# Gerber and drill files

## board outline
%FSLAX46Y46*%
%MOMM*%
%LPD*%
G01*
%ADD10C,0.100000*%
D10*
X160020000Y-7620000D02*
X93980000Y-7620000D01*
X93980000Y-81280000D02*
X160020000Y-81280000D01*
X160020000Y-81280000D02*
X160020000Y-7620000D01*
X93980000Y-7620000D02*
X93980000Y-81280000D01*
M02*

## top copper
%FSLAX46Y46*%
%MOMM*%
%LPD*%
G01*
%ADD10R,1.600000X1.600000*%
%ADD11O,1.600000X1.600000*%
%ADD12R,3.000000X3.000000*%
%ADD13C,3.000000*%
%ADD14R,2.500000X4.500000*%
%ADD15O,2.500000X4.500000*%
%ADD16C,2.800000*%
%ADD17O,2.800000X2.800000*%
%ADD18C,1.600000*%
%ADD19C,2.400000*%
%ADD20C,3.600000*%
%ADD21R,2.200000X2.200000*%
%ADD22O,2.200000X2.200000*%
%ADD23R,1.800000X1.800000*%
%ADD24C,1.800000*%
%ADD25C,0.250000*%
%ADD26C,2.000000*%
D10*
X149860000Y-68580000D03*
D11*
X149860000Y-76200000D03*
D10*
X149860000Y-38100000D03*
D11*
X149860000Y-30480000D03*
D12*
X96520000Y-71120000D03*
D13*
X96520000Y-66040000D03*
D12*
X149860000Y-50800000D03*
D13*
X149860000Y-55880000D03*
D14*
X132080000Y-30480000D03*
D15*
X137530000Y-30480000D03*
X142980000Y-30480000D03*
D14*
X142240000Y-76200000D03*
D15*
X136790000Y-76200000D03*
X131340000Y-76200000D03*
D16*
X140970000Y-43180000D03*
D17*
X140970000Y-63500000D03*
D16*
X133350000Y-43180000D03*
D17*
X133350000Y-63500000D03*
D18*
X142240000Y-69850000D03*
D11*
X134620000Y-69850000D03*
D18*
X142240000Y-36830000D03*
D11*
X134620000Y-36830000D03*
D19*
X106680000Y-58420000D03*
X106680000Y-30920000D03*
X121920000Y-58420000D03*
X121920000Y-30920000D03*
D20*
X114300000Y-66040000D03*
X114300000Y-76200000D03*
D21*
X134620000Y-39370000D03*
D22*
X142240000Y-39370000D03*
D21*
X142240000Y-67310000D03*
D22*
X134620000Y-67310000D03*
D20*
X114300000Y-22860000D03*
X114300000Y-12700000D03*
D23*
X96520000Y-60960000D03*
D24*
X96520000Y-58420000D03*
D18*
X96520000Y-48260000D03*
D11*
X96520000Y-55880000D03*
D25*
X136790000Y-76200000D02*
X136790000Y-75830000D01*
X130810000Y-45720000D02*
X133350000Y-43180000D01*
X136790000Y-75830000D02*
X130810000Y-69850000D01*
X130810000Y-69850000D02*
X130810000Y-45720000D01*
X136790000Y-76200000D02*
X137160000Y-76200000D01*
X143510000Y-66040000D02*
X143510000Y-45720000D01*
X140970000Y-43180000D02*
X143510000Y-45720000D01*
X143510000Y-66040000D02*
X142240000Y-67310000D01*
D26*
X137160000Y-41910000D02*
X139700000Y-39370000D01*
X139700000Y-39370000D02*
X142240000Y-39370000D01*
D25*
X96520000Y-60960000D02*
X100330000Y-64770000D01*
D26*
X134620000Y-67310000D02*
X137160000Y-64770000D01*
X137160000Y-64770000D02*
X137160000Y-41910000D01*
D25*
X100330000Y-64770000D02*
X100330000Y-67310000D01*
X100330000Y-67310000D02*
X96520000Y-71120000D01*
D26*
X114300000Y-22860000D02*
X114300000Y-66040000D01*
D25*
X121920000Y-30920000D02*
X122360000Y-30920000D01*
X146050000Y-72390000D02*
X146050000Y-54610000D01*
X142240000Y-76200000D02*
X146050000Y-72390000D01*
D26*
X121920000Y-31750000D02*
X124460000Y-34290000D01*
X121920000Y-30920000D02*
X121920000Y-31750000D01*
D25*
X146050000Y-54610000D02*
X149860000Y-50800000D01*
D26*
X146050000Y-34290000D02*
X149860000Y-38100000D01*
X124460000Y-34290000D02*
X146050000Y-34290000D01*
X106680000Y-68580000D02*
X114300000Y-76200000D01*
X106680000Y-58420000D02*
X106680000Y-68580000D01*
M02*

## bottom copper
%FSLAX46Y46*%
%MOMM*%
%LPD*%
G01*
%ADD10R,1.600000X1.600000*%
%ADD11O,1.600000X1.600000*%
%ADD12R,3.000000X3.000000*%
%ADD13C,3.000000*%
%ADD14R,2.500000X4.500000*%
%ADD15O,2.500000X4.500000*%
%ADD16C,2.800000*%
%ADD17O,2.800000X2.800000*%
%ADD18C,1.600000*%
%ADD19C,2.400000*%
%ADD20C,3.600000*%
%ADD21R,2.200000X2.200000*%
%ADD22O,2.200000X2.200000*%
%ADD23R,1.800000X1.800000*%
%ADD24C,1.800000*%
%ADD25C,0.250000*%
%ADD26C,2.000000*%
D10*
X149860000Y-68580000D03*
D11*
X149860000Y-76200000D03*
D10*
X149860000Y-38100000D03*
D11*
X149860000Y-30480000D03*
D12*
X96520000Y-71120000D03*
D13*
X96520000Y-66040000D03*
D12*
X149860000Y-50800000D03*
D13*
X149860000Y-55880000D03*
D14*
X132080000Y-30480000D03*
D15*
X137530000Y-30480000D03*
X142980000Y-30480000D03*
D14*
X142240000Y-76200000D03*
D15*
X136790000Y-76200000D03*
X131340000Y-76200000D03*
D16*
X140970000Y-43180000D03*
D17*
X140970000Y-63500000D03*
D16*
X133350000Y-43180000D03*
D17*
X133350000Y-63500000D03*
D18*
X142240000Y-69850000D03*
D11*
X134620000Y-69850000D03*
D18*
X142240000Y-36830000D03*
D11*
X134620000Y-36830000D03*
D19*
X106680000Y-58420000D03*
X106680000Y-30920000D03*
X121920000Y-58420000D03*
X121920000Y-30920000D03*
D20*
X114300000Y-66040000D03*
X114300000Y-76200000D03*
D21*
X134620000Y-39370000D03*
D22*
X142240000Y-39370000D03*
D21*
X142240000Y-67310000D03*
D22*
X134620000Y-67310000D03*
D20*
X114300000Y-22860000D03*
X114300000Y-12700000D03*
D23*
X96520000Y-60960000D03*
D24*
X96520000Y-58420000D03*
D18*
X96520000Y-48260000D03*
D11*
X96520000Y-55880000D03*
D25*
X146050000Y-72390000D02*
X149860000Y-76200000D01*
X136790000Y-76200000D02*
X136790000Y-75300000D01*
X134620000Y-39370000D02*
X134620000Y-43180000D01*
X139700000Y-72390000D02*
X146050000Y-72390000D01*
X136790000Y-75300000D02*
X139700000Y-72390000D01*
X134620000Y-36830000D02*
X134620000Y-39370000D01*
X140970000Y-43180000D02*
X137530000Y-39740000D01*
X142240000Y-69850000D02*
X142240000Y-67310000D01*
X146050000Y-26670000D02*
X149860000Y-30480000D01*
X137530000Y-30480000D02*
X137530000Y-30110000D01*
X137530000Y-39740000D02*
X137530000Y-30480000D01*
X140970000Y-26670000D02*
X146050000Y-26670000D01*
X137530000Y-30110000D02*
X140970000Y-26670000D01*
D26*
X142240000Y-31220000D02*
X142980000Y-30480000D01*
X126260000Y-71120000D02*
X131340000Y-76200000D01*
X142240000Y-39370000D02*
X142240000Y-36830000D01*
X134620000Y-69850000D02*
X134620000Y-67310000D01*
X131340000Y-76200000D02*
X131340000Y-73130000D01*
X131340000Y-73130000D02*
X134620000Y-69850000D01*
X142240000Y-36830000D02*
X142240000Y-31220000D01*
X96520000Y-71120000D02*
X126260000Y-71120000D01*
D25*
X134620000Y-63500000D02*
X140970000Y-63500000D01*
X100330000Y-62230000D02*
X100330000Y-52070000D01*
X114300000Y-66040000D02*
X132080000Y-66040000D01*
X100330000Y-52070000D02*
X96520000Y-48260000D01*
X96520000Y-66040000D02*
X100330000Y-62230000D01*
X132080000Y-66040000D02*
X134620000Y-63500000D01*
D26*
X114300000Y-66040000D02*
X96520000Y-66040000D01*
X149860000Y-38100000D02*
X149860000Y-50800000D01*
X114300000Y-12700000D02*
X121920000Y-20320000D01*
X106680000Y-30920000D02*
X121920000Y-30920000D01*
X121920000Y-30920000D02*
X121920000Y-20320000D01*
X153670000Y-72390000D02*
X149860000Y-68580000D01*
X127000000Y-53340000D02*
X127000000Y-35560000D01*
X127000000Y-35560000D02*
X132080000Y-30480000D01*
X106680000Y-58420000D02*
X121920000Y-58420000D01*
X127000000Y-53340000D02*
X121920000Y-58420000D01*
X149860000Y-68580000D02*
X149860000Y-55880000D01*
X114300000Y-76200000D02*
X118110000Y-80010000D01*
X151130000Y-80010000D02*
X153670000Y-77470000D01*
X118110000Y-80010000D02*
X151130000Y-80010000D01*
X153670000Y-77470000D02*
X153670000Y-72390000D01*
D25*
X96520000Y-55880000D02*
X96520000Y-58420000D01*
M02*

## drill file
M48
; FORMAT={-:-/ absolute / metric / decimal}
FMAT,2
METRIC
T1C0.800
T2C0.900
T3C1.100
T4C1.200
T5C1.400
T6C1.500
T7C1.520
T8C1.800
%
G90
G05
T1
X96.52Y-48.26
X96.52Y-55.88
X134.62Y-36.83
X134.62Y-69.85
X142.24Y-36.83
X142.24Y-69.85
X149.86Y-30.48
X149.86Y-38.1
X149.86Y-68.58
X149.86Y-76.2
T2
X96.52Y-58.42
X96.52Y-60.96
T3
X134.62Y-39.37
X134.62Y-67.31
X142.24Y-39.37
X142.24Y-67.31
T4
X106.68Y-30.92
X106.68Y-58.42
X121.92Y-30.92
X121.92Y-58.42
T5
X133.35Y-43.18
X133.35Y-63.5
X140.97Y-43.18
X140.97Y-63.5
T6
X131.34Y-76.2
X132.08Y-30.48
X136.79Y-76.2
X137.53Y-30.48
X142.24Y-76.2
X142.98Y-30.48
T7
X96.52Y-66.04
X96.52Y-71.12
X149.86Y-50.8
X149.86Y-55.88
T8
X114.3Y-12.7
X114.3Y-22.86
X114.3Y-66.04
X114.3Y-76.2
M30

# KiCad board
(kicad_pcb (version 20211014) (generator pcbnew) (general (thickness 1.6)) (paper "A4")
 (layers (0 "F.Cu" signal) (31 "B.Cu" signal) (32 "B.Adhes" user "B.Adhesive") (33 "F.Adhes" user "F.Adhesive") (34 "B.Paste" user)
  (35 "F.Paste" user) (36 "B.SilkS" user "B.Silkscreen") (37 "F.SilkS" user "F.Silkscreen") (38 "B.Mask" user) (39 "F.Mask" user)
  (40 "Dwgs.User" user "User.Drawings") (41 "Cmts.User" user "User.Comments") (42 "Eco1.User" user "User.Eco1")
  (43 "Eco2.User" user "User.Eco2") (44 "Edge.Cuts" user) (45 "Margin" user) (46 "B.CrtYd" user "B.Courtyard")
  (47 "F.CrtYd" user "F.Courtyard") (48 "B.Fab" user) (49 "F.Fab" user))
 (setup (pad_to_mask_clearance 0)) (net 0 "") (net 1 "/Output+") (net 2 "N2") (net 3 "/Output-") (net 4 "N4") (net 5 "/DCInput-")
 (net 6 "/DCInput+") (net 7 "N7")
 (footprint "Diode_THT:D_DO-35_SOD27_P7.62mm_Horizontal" (layer "F.Cu") (at 149.86 68.58 -90)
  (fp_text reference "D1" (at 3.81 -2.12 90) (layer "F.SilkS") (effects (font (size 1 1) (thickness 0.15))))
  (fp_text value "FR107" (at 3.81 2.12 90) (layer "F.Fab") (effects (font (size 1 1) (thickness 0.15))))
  (pad "1" thru_hole rect (at 0 0 270) (size 1.6 1.6) (drill 0.8) (layers *.Cu *.Mask) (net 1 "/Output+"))
  (pad "2" thru_hole oval (at 7.62 0 270) (size 1.6 1.6) (drill 0.8) (layers *.Cu *.Mask) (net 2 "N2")))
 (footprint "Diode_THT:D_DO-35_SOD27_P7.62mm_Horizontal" (layer "F.Cu") (at 149.86 38.1 90)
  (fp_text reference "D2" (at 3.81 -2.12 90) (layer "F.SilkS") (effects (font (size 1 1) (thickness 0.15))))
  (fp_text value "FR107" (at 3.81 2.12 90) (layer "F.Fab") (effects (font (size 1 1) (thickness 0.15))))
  (pad "1" thru_hole rect (at 0 0 90) (size 1.6 1.6) (drill 0.8) (layers *.Cu *.Mask) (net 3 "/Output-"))
  (pad "2" thru_hole oval (at 7.62 0 90) (size 1.6 1.6) (drill 0.8) (layers *.Cu *.Mask) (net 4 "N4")))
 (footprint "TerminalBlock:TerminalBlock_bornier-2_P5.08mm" (layer "F.Cu") (at 96.52 71.12 90)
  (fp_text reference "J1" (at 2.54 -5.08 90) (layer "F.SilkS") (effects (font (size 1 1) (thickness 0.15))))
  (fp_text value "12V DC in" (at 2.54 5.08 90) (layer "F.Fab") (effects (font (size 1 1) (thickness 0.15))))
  (pad "1" thru_hole rect (at 0 0 90) (size 3 3) (drill 1.52) (layers *.Cu *.Mask) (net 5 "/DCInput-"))
  (pad "2" thru_hole circle (at 5.08 0 90) (size 3 3) (drill 1.52) (layers *.Cu *.Mask) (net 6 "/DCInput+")))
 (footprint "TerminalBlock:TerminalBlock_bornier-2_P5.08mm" (layer "F.Cu") (at 149.86 50.8 -90)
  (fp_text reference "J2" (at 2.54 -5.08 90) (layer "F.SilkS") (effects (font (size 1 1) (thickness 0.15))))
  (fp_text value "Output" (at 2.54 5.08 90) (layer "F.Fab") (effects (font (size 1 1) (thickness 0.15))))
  (pad "1" thru_hole rect (at 0 0 270) (size 3 3) (drill 1.52) (layers *.Cu *.Mask) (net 3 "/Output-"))
  (pad "2" thru_hole circle (at 5.08 0 270) (size 3 3) (drill 1.52) (layers *.Cu *.Mask) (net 1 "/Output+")))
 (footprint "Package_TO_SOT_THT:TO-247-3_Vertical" (layer "F.Cu") (at 132.08 30.48)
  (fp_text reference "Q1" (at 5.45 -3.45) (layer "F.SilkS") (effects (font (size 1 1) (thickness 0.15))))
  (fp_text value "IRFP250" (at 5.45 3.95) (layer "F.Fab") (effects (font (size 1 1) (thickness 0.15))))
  (pad "1" thru_hole rect (at 0 0) (size 2.5 4.5) (drill 1.5) (layers *.Cu *.Mask) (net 1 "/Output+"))
  (pad "2" thru_hole oval (at 5.45 0) (size 2.5 4.5) (drill 1.5) (layers *.Cu *.Mask) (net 4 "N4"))
  (pad "3" thru_hole oval (at 10.9 0) (size 2.5 4.5) (drill 1.5) (layers *.Cu *.Mask) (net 5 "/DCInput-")))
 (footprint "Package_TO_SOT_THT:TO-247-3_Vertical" (layer "F.Cu") (at 142.24 76.2 180)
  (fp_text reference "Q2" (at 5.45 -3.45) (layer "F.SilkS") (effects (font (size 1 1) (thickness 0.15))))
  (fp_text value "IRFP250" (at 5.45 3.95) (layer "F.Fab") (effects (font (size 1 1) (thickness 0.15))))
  (pad "1" thru_hole rect (at 0 0 180) (size 2.5 4.5) (drill 1.5) (layers *.Cu *.Mask) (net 3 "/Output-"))
  (pad "2" thru_hole oval (at 5.45 0 180) (size 2.5 4.5) (drill 1.5) (layers *.Cu *.Mask) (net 2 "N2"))
  (pad "3" thru_hole oval (at 10.9 0 180) (size 2.5 4.5) (drill 1.5) (layers *.Cu *.Mask) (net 5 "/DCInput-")))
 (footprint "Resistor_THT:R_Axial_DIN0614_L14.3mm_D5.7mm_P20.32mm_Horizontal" (layer "F.Cu") (at 140.97 43.18 -90)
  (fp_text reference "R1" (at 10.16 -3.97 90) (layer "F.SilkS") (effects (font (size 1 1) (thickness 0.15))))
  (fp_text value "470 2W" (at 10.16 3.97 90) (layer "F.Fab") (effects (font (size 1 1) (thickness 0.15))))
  (pad "1" thru_hole circle (at 0 0 270) (size 2.8 2.8) (drill 1.4) (layers *.Cu *.Mask) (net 4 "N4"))
  (pad "2" thru_hole oval (at 20.32 0 270) (size 2.8 2.8) (drill 1.4) (layers *.Cu *.Mask) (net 6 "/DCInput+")))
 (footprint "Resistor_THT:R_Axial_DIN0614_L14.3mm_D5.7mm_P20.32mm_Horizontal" (layer "F.Cu") (at 133.35 43.18 -90)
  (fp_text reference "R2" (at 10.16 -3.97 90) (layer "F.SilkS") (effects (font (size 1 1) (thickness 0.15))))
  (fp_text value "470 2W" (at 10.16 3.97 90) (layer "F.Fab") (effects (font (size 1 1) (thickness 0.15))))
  (pad "1" thru_hole circle (at 0 0 270) (size 2.8 2.8) (drill 1.4) (layers *.Cu *.Mask) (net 2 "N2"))
  (pad "2" thru_hole oval (at 20.32 0 270) (size 2.8 2.8) (drill 1.4) (layers *.Cu *.Mask) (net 6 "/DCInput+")))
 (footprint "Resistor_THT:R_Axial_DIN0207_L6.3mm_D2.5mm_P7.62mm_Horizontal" (layer "F.Cu") (at 142.24 69.85 180)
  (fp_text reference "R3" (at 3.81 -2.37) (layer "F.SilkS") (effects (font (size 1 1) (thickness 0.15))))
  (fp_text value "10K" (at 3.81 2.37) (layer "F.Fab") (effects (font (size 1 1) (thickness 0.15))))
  (pad "1" thru_hole circle (at 0 0 180) (size 1.6 1.6) (drill 0.8) (layers *.Cu *.Mask) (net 4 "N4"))
  (pad "2" thru_hole oval (at 7.62 0 180) (size 1.6 1.6) (drill 0.8) (layers *.Cu *.Mask) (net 5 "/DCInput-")))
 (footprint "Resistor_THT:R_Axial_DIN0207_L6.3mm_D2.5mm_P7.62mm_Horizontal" (layer "F.Cu") (at 142.24 36.83 180)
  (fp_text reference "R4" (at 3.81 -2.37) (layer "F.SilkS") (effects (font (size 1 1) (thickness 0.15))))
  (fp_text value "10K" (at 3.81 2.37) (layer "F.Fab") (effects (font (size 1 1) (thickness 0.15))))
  (pad "1" thru_hole circle (at 0 0 180) (size 1.6 1.6) (drill 0.8) (layers *.Cu *.Mask) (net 5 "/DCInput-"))
  (pad "2" thru_hole oval (at 7.62 0 180) (size 1.6 1.6) (drill 0.8) (layers *.Cu *.Mask) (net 2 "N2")))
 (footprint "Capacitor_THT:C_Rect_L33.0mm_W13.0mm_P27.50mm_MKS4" (layer "F.Cu") (at 106.68 58.42 90)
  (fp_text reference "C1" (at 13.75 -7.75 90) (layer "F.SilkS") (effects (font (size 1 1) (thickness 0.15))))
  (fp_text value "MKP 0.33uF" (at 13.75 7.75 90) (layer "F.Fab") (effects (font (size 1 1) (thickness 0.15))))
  (pad "1" thru_hole circle (at 0 0 90) (size 2.4 2.4) (drill 1.2) (layers *.Cu *.Mask) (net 1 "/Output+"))
  (pad "2" thru_hole circle (at 27.5 0 90) (size 2.4 2.4) (drill 1.2) (layers *.Cu *.Mask) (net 3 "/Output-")))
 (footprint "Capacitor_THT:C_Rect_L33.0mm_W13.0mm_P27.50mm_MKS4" (layer "F.Cu") (at 121.92 58.42 90)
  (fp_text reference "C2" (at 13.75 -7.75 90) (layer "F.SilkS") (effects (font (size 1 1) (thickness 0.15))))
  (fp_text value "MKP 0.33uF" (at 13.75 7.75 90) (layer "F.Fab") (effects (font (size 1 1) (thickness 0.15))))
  (pad "1" thru_hole circle (at 0 0 90) (size 2.4 2.4) (drill 1.2) (layers *.Cu *.Mask) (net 1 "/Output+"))
  (pad "2" thru_hole circle (at 27.5 0 90) (size 2.4 2.4) (drill 1.2) (layers *.Cu *.Mask) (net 3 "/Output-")))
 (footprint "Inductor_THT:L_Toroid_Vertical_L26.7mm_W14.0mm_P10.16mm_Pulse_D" (layer "F.Cu") (at 114.3 66.04)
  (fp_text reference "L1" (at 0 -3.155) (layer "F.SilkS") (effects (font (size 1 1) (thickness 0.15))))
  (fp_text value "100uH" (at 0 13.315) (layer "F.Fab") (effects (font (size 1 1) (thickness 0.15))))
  (pad "1" thru_hole circle (at 0 0) (size 3.6 3.6) (drill 1.8) (layers *.Cu *.Mask) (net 6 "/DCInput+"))
  (pad "2" thru_hole circle (at 0 10.16) (size 3.6 3.6) (drill 1.8) (layers *.Cu *.Mask) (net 1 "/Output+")))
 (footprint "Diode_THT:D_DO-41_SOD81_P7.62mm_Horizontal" (layer "F.Cu") (at 134.62 39.37)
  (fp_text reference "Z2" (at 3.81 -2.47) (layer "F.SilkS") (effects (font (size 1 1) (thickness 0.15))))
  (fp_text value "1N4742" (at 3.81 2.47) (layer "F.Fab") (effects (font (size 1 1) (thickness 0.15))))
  (pad "1" thru_hole rect (at 0 0) (size 2.2 2.2) (drill 1.1) (layers *.Cu *.Mask) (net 2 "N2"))
  (pad "2" thru_hole oval (at 7.62 0) (size 2.2 2.2) (drill 1.1) (layers *.Cu *.Mask) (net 5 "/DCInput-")))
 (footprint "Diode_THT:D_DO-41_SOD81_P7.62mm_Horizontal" (layer "F.Cu") (at 142.24 67.31 180)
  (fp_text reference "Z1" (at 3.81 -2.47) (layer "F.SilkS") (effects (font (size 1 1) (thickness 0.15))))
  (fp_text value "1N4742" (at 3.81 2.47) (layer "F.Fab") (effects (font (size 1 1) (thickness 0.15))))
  (pad "1" thru_hole rect (at 0 0 180) (size 2.2 2.2) (drill 1.1) (layers *.Cu *.Mask) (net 4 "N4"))
  (pad "2" thru_hole oval (at 7.62 0 180) (size 2.2 2.2) (drill 1.1) (layers *.Cu *.Mask) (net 5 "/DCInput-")))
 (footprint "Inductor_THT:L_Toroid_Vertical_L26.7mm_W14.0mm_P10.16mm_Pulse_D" (layer "F.Cu") (at 114.3 22.86 180)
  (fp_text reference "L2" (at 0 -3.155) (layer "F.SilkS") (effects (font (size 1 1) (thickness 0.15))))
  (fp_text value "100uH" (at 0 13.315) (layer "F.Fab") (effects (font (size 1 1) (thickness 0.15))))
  (pad "1" thru_hole circle (at 0 0 180) (size 3.6 3.6) (drill 1.8) (layers *.Cu *.Mask) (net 6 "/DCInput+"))
  (pad "2" thru_hole circle (at 0 10.16 180) (size 3.6 3.6) (drill 1.8) (layers *.Cu *.Mask) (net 3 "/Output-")))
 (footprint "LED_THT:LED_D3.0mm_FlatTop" (layer "F.Cu") (at 96.52 60.96 90)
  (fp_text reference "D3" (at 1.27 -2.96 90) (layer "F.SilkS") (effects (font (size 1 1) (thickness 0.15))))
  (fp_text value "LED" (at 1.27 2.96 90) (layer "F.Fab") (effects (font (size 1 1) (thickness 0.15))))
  (pad "1" thru_hole rect (at 0 0 90) (size 1.8 1.8) (drill 0.9) (layers *.Cu *.Mask) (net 5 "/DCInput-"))
  (pad "2" thru_hole circle (at 2.54 0 90) (size 1.8 1.8) (drill 0.9) (layers *.Cu *.Mask) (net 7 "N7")))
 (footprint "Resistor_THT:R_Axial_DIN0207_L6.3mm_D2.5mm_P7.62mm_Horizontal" (layer "F.Cu") (at 96.52 48.26 -90)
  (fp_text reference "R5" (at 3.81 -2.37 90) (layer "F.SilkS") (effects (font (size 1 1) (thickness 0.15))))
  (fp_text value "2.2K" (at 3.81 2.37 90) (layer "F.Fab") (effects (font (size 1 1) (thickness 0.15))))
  (pad "1" thru_hole circle (at 0 0 270) (size 1.6 1.6) (drill 0.8) (layers *.Cu *.Mask) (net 6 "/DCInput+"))
  (pad "2" thru_hole oval (at 7.62 0 270) (size 1.6 1.6) (drill 0.8) (layers *.Cu *.Mask) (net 7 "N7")))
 (gr_line (start 160.02 7.62) (end 93.98 7.62) (layer "Edge.Cuts") (width 0.1))
 (gr_line (start 93.98 81.28) (end 160.02 81.28) (layer "Edge.Cuts") (width 0.1))
 (gr_line (start 160.02 81.28) (end 160.02 7.62) (layer "Edge.Cuts") (width 0.1))
 (gr_line (start 93.98 7.62) (end 93.98 81.28) (layer "Edge.Cuts") (width 0.1))
 (segment (start 136.79 76.2) (end 136.79 75.83) (width 0.25) (layer "F.Cu") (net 2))
 (segment (start 130.81 45.72) (end 133.35 43.18) (width 0.25) (layer "F.Cu") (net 2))
 (segment (start 136.79 75.83) (end 130.81 69.85) (width 0.25) (layer "F.Cu") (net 2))
 (segment (start 130.81 69.85) (end 130.81 45.72) (width 0.25) (layer "F.Cu") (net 2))
 (segment (start 136.79 76.2) (end 137.16 76.2) (width 0.25) (layer "F.Cu") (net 2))
 (segment (start 146.05 72.39) (end 149.86 76.2) (width 0.25) (layer "B.Cu") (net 2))
 (segment (start 136.79 76.2) (end 136.79 75.3) (width 0.25) (layer "B.Cu") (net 2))
 (segment (start 134.62 39.37) (end 134.62 43.18) (width 0.25) (layer "B.Cu") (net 2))
 (segment (start 139.7 72.39) (end 146.05 72.39) (width 0.25) (layer "B.Cu") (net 2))
 (segment (start 136.79 75.3) (end 139.7 72.39) (width 0.25) (layer "B.Cu") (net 2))
 (segment (start 134.62 36.83) (end 134.62 39.37) (width 0.25) (layer "B.Cu") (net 2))
 (segment (start 143.51 66.04) (end 143.51 45.72) (width 0.25) (layer "F.Cu") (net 4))
 (segment (start 140.97 43.18) (end 143.51 45.72) (width 0.25) (layer "F.Cu") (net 4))
 (segment (start 143.51 66.04) (end 142.24 67.31) (width 0.25) (layer "F.Cu") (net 4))
 (segment (start 140.97 43.18) (end 137.53 39.74) (width 0.25) (layer "B.Cu") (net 4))
 (segment (start 142.24 69.85) (end 142.24 67.31) (width 0.25) (layer "B.Cu") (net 4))
 (segment (start 146.05 26.67) (end 149.86 30.48) (width 0.25) (layer "B.Cu") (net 4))
 (segment (start 137.53 30.48) (end 137.53 30.11) (width 0.25) (layer "B.Cu") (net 4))
 (segment (start 137.53 39.74) (end 137.53 30.48) (width 0.25) (layer "B.Cu") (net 4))
 (segment (start 140.97 26.67) (end 146.05 26.67) (width 0.25) (layer "B.Cu") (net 4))
 (segment (start 137.53 30.11) (end 140.97 26.67) (width 0.25) (layer "B.Cu") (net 4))
 (segment (start 137.16 41.91) (end 139.7 39.37) (width 2) (layer "F.Cu") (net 5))
 (segment (start 139.7 39.37) (end 142.24 39.37) (width 2) (layer "F.Cu") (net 5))
 (segment (start 96.52 60.96) (end 100.33 64.77) (width 0.25) (layer "F.Cu") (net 5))
 (segment (start 134.62 67.31) (end 137.16 64.77) (width 2) (layer "F.Cu") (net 5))
 (segment (start 137.16 64.77) (end 137.16 41.91) (width 2) (layer "F.Cu") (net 5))
 (segment (start 100.33 64.77) (end 100.33 67.31) (width 0.25) (layer "F.Cu") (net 5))
 (segment (start 100.33 67.31) (end 96.52 71.12) (width 0.25) (layer "F.Cu") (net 5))
 (segment (start 142.24 31.22) (end 142.98 30.48) (width 2) (layer "B.Cu") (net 5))
 (segment (start 126.26 71.12) (end 131.34 76.2) (width 2) (layer "B.Cu") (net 5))
 (segment (start 142.24 39.37) (end 142.24 36.83) (width 2) (layer "B.Cu") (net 5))
 (segment (start 134.62 69.85) (end 134.62 67.31) (width 2) (layer "B.Cu") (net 5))
 (segment (start 131.34 76.2) (end 131.34 73.13) (width 2) (layer "B.Cu") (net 5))
 (segment (start 131.34 73.13) (end 134.62 69.85) (width 2) (layer "B.Cu") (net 5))
 (segment (start 142.24 36.83) (end 142.24 31.22) (width 2) (layer "B.Cu") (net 5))
 (segment (start 96.52 71.12) (end 126.26 71.12) (width 2) (layer "B.Cu") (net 5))
 (segment (start 114.3 22.86) (end 114.3 66.04) (width 2) (layer "F.Cu") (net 6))
 (segment (start 134.62 63.5) (end 140.97 63.5) (width 0.25) (layer "B.Cu") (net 6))
 (segment (start 100.33 62.23) (end 100.33 52.07) (width 0.25) (layer "B.Cu") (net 6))
 (segment (start 114.3 66.04) (end 132.08 66.04) (width 0.25) (layer "B.Cu") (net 6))
 (segment (start 100.33 52.07) (end 96.52 48.26) (width 0.25) (layer "B.Cu") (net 6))
 (segment (start 96.52 66.04) (end 100.33 62.23) (width 0.25) (layer "B.Cu") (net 6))
 (segment (start 132.08 66.04) (end 134.62 63.5) (width 0.25) (layer "B.Cu") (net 6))
 (segment (start 114.3 66.04) (end 96.52 66.04) (width 2) (layer "B.Cu") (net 6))
 (segment (start 121.92 30.92) (end 122.36 30.92) (width 0.25) (layer "F.Cu") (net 3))
 (segment (start 146.05 72.39) (end 146.05 54.61) (width 0.25) (layer "F.Cu") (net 3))
 (segment (start 142.24 76.2) (end 146.05 72.39) (width 0.25) (layer "F.Cu") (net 3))
 (segment (start 121.92 31.75) (end 124.46 34.29) (width 2) (layer "F.Cu") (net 3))
 (segment (start 121.92 30.92) (end 121.92 31.75) (width 2) (layer "F.Cu") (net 3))
 (segment (start 146.05 54.61) (end 149.86 50.8) (width 0.25) (layer "F.Cu") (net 3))
 (segment (start 146.05 34.29) (end 149.86 38.1) (width 2) (layer "F.Cu") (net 3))
 (segment (start 124.46 34.29) (end 146.05 34.29) (width 2) (layer "F.Cu") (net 3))
 (segment (start 149.86 38.1) (end 149.86 50.8) (width 2) (layer "B.Cu") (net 3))
 (segment (start 114.3 12.7) (end 121.92 20.32) (width 2) (layer "B.Cu") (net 3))
 (segment (start 106.68 30.92) (end 121.92 30.92) (width 2) (layer "B.Cu") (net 3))
 (segment (start 121.92 30.92) (end 121.92 20.32) (width 2) (layer "B.Cu") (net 3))
 (segment (start 106.68 68.58) (end 114.3 76.2) (width 2) (layer "F.Cu") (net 1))
 (segment (start 106.68 58.42) (end 106.68 68.58) (width 2) (layer "F.Cu") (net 1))
 (segment (start 153.67 72.39) (end 149.86 68.58) (width 2) (layer "B.Cu") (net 1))
 (segment (start 127 53.34) (end 127 35.56) (width 2) (layer "B.Cu") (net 1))
 (segment (start 127 35.56) (end 132.08 30.48) (width 2) (layer "B.Cu") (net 1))
 (segment (start 106.68 58.42) (end 121.92 58.42) (width 2) (layer "B.Cu") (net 1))
 (segment (start 127 53.34) (end 121.92 58.42) (width 2) (layer "B.Cu") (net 1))
 (segment (start 149.86 68.58) (end 149.86 55.88) (width 2) (layer "B.Cu") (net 1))
 (segment (start 114.3 76.2) (end 118.11 80.01) (width 2) (layer "B.Cu") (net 1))
 (segment (start 151.13 80.01) (end 153.67 77.47) (width 2) (layer "B.Cu") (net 1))
 (segment (start 118.11 80.01) (end 151.13 80.01) (width 2) (layer "B.Cu") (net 1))
 (segment (start 153.67 77.47) (end 153.67 72.39) (width 2) (layer "B.Cu") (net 1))
 (segment (start 96.52 55.88) (end 96.52 58.42) (width 0.25) (layer "B.Cu") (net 7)))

